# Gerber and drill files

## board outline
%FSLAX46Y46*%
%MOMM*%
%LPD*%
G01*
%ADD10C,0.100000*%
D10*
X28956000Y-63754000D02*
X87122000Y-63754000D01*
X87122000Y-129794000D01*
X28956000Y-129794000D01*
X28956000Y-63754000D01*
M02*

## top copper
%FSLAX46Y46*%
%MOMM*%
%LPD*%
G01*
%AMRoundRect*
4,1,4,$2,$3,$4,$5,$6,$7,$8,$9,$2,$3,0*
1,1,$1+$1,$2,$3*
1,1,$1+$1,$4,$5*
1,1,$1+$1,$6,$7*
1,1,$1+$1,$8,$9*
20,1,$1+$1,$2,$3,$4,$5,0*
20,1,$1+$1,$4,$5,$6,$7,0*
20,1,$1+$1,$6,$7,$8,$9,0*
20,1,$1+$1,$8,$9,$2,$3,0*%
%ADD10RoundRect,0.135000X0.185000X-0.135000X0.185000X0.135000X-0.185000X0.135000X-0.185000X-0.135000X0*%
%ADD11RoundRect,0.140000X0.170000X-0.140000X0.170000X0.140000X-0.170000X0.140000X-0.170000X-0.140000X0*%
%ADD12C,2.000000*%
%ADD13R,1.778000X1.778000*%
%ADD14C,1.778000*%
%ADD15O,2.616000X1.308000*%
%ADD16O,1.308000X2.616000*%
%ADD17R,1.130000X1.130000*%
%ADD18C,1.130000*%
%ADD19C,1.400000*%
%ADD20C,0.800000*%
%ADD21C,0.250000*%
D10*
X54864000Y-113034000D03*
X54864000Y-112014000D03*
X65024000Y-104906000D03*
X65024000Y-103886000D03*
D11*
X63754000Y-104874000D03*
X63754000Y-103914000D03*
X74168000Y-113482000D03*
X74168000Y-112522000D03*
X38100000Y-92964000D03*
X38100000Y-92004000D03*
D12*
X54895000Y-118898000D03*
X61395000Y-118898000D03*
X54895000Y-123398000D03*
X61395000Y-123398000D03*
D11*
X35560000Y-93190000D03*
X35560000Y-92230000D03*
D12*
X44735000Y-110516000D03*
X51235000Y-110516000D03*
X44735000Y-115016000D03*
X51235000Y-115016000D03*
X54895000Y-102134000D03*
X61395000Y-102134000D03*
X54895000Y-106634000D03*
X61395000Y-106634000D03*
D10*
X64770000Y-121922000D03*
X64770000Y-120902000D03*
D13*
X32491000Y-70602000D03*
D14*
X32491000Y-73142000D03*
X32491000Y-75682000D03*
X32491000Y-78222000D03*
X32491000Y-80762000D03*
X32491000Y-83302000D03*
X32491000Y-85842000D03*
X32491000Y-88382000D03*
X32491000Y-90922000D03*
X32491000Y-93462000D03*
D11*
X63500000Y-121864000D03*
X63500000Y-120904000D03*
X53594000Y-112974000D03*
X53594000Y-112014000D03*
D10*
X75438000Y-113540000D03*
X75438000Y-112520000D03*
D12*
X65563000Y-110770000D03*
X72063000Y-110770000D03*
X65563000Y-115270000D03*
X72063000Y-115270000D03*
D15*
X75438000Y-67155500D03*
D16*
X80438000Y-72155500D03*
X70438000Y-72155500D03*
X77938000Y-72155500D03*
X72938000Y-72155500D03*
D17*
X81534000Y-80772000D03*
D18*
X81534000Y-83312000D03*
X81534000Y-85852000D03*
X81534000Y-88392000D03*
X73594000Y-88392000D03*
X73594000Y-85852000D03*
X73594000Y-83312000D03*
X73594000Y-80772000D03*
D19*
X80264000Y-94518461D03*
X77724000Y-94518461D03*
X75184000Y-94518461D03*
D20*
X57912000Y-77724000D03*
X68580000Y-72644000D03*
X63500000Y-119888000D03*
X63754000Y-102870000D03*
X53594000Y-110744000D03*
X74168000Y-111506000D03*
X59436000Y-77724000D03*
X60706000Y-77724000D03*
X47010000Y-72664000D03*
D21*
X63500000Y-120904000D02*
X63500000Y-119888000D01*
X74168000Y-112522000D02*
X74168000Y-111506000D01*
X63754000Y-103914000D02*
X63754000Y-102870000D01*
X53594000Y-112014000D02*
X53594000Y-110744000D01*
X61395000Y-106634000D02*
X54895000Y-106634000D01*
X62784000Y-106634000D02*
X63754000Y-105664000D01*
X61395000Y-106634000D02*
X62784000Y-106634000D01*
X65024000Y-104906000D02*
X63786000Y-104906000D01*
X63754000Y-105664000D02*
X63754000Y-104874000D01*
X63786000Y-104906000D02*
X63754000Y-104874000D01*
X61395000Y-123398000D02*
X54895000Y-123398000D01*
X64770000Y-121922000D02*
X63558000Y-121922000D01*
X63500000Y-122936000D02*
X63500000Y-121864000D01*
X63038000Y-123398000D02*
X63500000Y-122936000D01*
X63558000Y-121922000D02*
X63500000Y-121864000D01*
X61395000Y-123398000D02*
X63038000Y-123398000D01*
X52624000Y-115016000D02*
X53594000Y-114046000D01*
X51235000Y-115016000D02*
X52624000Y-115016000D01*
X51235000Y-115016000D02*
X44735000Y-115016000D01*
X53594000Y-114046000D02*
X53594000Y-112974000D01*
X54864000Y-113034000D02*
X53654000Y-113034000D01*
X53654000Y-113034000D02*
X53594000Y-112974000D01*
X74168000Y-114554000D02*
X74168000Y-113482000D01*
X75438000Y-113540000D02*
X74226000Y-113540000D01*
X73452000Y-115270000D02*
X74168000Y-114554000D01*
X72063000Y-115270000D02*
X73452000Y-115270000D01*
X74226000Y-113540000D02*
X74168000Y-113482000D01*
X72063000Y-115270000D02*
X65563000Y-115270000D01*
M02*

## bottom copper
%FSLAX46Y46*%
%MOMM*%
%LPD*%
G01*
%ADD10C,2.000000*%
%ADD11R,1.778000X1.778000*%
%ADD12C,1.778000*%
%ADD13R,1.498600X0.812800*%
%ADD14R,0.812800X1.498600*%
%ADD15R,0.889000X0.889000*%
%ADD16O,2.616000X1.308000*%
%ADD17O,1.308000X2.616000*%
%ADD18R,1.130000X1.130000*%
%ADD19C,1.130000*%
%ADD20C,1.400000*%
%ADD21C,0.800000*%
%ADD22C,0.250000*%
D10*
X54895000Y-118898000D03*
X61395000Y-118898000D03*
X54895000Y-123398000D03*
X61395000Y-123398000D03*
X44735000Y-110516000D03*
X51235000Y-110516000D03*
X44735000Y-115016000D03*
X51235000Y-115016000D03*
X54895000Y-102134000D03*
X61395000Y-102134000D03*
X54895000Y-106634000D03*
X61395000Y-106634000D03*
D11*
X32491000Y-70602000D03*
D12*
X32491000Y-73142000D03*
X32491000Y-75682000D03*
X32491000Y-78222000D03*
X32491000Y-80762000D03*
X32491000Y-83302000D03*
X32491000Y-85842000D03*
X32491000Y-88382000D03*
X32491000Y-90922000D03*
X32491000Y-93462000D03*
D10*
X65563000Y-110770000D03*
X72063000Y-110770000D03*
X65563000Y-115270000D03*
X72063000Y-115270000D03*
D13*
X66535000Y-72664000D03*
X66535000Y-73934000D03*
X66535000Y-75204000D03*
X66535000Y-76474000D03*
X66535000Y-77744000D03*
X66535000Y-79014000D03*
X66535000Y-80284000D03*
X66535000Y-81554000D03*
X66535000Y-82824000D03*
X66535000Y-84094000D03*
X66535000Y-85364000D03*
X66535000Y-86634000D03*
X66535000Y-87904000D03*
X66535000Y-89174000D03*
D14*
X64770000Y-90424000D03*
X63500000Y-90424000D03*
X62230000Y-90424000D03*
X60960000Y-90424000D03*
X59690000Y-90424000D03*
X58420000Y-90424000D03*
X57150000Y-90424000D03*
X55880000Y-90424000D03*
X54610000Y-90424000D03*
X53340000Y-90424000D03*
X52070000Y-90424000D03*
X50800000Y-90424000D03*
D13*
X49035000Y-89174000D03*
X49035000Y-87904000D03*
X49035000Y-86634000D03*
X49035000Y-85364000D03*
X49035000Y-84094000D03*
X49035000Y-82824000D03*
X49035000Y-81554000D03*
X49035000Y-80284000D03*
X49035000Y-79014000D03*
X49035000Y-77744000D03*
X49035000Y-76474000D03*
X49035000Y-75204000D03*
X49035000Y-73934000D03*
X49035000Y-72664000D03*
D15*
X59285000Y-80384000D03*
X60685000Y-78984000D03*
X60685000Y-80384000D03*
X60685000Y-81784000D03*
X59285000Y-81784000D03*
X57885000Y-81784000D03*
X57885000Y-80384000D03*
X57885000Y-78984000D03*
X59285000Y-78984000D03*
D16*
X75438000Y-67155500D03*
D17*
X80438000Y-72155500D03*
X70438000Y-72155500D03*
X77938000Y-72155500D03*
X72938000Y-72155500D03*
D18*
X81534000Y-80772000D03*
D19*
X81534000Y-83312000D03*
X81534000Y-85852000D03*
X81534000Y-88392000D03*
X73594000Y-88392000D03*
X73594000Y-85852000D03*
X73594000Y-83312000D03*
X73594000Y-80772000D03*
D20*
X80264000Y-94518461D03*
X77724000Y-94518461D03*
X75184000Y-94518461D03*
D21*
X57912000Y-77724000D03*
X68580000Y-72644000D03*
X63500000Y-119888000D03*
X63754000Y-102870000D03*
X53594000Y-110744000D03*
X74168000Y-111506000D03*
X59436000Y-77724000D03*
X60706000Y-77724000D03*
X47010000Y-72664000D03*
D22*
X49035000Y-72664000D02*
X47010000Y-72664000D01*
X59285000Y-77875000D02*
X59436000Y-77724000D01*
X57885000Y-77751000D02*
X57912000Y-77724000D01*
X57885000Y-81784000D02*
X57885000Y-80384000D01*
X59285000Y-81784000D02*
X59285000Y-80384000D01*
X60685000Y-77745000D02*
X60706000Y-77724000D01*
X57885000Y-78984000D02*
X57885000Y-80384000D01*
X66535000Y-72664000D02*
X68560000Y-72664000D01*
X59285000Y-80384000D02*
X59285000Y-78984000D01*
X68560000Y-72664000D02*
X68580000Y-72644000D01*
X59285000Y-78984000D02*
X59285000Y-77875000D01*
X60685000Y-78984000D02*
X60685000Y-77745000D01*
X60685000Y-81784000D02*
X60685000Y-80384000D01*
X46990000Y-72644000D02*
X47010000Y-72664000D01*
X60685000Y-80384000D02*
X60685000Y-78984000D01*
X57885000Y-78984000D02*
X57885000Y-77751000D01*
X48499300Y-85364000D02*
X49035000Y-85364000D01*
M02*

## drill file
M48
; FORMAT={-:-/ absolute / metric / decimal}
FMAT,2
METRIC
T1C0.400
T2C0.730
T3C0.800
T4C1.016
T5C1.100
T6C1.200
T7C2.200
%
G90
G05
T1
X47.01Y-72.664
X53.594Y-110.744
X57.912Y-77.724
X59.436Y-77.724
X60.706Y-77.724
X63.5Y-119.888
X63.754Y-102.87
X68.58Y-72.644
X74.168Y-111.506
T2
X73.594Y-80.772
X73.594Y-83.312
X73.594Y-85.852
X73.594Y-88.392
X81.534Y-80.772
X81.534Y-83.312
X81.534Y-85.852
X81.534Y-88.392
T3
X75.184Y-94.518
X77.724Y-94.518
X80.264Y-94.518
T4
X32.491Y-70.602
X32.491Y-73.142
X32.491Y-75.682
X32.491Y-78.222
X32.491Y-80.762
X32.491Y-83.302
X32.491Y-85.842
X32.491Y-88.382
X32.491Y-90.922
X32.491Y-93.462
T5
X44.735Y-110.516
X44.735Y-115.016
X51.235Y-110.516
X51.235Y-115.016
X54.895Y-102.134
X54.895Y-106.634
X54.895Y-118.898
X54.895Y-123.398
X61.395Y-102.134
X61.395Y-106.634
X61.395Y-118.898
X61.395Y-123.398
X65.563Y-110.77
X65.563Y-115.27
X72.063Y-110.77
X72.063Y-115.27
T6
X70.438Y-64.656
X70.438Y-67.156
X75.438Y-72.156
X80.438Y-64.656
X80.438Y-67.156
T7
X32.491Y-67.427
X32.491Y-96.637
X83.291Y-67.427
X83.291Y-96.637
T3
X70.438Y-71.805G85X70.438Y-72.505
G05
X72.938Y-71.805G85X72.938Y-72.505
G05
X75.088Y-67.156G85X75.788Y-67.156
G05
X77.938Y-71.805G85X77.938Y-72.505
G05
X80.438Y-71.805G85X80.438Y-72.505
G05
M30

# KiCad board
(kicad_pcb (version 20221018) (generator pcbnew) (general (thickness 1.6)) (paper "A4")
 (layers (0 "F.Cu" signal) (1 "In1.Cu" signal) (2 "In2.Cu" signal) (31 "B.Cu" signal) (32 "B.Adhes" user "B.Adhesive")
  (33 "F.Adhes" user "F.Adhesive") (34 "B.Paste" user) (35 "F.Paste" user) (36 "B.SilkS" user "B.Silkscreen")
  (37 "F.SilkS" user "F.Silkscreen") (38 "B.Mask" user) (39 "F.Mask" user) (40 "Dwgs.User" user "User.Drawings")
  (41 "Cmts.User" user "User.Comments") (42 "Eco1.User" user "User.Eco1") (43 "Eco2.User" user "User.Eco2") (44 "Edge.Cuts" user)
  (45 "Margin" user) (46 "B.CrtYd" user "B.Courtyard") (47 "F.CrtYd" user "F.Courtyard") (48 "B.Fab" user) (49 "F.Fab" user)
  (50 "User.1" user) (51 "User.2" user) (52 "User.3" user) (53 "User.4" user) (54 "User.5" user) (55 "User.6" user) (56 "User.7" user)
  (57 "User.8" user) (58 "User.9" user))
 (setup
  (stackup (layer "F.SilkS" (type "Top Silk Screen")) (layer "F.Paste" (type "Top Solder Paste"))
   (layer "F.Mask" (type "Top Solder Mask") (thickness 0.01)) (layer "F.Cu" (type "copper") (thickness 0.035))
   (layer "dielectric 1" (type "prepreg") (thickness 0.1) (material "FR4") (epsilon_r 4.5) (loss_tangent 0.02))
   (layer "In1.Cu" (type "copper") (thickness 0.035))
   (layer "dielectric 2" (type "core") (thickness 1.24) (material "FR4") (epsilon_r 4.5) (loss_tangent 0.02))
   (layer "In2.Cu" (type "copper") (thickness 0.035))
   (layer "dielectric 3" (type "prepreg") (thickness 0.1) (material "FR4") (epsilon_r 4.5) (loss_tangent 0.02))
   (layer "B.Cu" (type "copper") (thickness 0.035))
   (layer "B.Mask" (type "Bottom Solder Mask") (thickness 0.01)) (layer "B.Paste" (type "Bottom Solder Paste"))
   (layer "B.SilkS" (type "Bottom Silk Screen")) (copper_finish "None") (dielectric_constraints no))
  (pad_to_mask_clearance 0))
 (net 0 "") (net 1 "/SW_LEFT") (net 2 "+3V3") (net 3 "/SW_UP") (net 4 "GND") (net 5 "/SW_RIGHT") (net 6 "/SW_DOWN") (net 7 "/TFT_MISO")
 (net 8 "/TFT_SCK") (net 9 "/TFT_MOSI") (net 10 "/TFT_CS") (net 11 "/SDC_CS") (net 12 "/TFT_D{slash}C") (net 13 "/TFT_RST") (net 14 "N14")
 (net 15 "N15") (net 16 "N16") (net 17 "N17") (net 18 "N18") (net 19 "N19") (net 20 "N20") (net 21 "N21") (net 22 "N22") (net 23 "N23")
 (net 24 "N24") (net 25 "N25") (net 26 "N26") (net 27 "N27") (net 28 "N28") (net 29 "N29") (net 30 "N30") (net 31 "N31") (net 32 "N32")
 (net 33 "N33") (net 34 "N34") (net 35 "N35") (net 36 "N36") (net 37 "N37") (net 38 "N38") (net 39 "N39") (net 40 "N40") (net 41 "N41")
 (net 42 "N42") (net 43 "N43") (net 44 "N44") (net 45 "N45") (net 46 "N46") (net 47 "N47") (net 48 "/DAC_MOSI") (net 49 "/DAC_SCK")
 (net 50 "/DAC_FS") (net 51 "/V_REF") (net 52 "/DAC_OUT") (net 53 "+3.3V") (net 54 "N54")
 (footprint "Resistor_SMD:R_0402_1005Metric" (layer "F.Cu") (at 54.864 112.524 90)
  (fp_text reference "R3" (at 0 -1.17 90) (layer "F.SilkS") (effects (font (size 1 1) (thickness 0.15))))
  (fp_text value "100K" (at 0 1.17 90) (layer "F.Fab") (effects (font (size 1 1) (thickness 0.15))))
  (pad "1" smd roundrect (at -0.51 0 90) (size 0.54 0.64) (layers "F.Cu" "F.Paste" "F.Mask") (roundrect_rratio 0.25) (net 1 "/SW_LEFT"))
  (pad "2" smd roundrect (at 0.51 0 90) (size 0.54 0.64) (layers "F.Cu" "F.Paste" "F.Mask") (roundrect_rratio 0.25) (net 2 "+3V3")))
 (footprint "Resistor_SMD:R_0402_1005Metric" (layer "F.Cu") (at 65.024 104.396 90)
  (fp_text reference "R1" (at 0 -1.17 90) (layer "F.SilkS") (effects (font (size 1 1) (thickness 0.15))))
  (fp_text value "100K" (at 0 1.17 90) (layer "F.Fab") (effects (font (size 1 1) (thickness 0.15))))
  (pad "1" smd roundrect (at -0.51 0 90) (size 0.54 0.64) (layers "F.Cu" "F.Paste" "F.Mask") (roundrect_rratio 0.25) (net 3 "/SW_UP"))
  (pad "2" smd roundrect (at 0.51 0 90) (size 0.54 0.64) (layers "F.Cu" "F.Paste" "F.Mask") (roundrect_rratio 0.25) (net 2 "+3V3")))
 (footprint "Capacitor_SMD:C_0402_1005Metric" (layer "F.Cu") (at 63.754 104.394 90)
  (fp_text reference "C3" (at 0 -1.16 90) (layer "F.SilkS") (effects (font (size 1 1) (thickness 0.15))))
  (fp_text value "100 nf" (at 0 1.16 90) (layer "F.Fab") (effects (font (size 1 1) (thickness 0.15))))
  (pad "1" smd roundrect (at -0.48 0 90) (size 0.56 0.62) (layers "F.Cu" "F.Paste" "F.Mask") (roundrect_rratio 0.25) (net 3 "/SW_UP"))
  (pad "2" smd roundrect (at 0.48 0 90) (size 0.56 0.62) (layers "F.Cu" "F.Paste" "F.Mask") (roundrect_rratio 0.25) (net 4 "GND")))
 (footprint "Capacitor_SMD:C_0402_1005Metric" (layer "F.Cu") (at 74.168 113.002 90)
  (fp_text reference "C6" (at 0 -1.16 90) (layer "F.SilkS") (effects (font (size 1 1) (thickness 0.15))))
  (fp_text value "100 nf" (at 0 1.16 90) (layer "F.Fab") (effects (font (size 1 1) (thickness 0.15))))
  (pad "1" smd roundrect (at -0.48 0 90) (size 0.56 0.62) (layers "F.Cu" "F.Paste" "F.Mask") (roundrect_rratio 0.25) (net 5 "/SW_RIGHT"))
  (pad "2" smd roundrect (at 0.48 0 90) (size 0.56 0.62) (layers "F.Cu" "F.Paste" "F.Mask") (roundrect_rratio 0.25) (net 4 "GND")))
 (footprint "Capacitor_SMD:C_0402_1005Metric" (layer "F.Cu") (at 38.1 92.484 90)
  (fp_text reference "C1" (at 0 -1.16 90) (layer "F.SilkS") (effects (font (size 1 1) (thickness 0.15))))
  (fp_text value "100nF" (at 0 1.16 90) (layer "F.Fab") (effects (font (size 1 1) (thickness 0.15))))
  (pad "1" smd roundrect (at -0.48 0 90) (size 0.56 0.62) (layers "F.Cu" "F.Paste" "F.Mask") (roundrect_rratio 0.25) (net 2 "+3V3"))
  (pad "2" smd roundrect (at 0.48 0 90) (size 0.56 0.62) (layers "F.Cu" "F.Paste" "F.Mask") (roundrect_rratio 0.25) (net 4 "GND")))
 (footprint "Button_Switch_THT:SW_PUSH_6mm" (layer "F.Cu") (at 54.895 118.898)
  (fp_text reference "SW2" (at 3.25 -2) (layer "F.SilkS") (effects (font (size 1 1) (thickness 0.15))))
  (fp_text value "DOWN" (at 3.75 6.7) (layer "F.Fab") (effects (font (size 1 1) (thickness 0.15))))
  (pad "1" thru_hole circle (at 0 0 90) (size 2 2) (drill 1.1) (layers "*.Cu" "*.Mask") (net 4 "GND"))
  (pad "1" thru_hole circle (at 6.5 0 90) (size 2 2) (drill 1.1) (layers "*.Cu" "*.Mask") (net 4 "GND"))
  (pad "2" thru_hole circle (at 0 4.5 90) (size 2 2) (drill 1.1) (layers "*.Cu" "*.Mask") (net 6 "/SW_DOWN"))
  (pad "2" thru_hole circle (at 6.5 4.5 90) (size 2 2) (drill 1.1) (layers "*.Cu" "*.Mask") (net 6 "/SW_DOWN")))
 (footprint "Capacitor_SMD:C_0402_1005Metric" (layer "F.Cu") (at 35.56 92.71 90)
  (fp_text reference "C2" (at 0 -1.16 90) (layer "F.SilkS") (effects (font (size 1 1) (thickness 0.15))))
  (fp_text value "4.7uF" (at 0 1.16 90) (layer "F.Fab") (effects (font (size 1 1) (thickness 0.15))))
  (pad "1" smd roundrect (at -0.48 0 90) (size 0.56 0.62) (layers "F.Cu" "F.Paste" "F.Mask") (roundrect_rratio 0.25) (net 2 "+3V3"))
  (pad "2" smd roundrect (at 0.48 0 90) (size 0.56 0.62) (layers "F.Cu" "F.Paste" "F.Mask") (roundrect_rratio 0.25) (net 4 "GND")))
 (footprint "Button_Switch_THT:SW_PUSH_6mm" (layer "F.Cu") (at 44.735 110.516)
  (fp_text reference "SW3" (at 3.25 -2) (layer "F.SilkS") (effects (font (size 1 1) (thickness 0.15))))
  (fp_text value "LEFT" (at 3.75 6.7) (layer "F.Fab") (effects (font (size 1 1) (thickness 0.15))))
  (pad "1" thru_hole circle (at 0 0 90) (size 2 2) (drill 1.1) (layers "*.Cu" "*.Mask") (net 4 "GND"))
  (pad "1" thru_hole circle (at 6.5 0 90) (size 2 2) (drill 1.1) (layers "*.Cu" "*.Mask") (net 4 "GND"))
  (pad "2" thru_hole circle (at 0 4.5 90) (size 2 2) (drill 1.1) (layers "*.Cu" "*.Mask") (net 1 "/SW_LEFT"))
  (pad "2" thru_hole circle (at 6.5 4.5 90) (size 2 2) (drill 1.1) (layers "*.Cu" "*.Mask") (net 1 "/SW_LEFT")))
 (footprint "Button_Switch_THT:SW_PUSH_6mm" (layer "F.Cu") (at 54.895 102.134)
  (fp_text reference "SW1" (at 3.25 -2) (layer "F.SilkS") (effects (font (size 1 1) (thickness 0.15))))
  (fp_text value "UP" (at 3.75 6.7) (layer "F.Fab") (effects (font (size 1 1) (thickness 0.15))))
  (pad "1" thru_hole circle (at 0 0 90) (size 2 2) (drill 1.1) (layers "*.Cu" "*.Mask") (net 4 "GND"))
  (pad "1" thru_hole circle (at 6.5 0 90) (size 2 2) (drill 1.1) (layers "*.Cu" "*.Mask") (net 4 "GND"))
  (pad "2" thru_hole circle (at 0 4.5 90) (size 2 2) (drill 1.1) (layers "*.Cu" "*.Mask") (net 3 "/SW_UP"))
  (pad "2" thru_hole circle (at 6.5 4.5 90) (size 2 2) (drill 1.1) (layers "*.Cu" "*.Mask") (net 3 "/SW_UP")))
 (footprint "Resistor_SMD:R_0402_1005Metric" (layer "F.Cu") (at 64.77 121.412 90)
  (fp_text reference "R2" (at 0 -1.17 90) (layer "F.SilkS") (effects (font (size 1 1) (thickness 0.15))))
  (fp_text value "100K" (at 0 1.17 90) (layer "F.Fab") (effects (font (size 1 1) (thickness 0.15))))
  (pad "1" smd roundrect (at -0.51 0 90) (size 0.54 0.64) (layers "F.Cu" "F.Paste" "F.Mask") (roundrect_rratio 0.25) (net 6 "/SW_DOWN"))
  (pad "2" smd roundrect (at 0.51 0 90) (size 0.54 0.64) (layers "F.Cu" "F.Paste" "F.Mask") (roundrect_rratio 0.25) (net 2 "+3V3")))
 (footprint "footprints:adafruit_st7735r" (layer "F.Cu") (at 57.891 82.032)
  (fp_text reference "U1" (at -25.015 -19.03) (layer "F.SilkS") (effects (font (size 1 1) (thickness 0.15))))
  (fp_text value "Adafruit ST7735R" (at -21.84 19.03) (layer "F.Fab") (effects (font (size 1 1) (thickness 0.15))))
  (pad "" np_thru_hole circle (at -25.4 -14.605) (size 2.2 2.2) (drill 2.2) (layers "*.Cu" "*.Mask"))
  (pad "" np_thru_hole circle (at -25.4 14.605) (size 2.2 2.2) (drill 2.2) (layers "*.Cu" "*.Mask"))
  (pad "" np_thru_hole circle (at 25.4 -14.605) (size 2.2 2.2) (drill 2.2) (layers "*.Cu" "*.Mask"))
  (pad "" np_thru_hole circle (at 25.4 14.605) (size 2.2 2.2) (drill 2.2) (layers "*.Cu" "*.Mask"))
  (pad "1" thru_hole rect (at -25.4 -11.43) (size 1.778 1.778) (drill 1.016) (layers "*.Cu" "*.Mask") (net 2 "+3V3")
   (solder_mask_margin 0.102))
  (pad "2" thru_hole circle (at -25.4 -8.89) (size 1.778 1.778) (drill 1.016) (layers "*.Cu" "*.Mask") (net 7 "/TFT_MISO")
   (solder_mask_margin 0.102))
  (pad "3" thru_hole circle (at -25.4 -6.35) (size 1.778 1.778) (drill 1.016) (layers "*.Cu" "*.Mask") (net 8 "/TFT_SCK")
   (solder_mask_margin 0.102))
  (pad "4" thru_hole circle (at -25.4 -3.81) (size 1.778 1.778) (drill 1.016) (layers "*.Cu" "*.Mask") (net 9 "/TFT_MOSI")
   (solder_mask_margin 0.102))
  (pad "5" thru_hole circle (at -25.4 -1.27) (size 1.778 1.778) (drill 1.016) (layers "*.Cu" "*.Mask") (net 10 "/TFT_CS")
   (solder_mask_margin 0.102))
  (pad "6" thru_hole circle (at -25.4 1.27) (size 1.778 1.778) (drill 1.016) (layers "*.Cu" "*.Mask") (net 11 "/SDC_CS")
   (solder_mask_margin 0.102))
  (pad "7" thru_hole circle (at -25.4 3.81) (size 1.778 1.778) (drill 1.016) (layers "*.Cu" "*.Mask") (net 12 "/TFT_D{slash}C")
   (solder_mask_margin 0.102))
  (pad "8" thru_hole circle (at -25.4 6.35) (size 1.778 1.778) (drill 1.016) (layers "*.Cu" "*.Mask") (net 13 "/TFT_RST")
   (solder_mask_margin 0.102))
  (pad "9" thru_hole circle (at -25.4 8.89) (size 1.778 1.778) (drill 1.016) (layers "*.Cu" "*.Mask") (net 2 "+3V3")
   (solder_mask_margin 0.102))
  (pad "10" thru_hole circle (at -25.4 11.43) (size 1.778 1.778) (drill 1.016) (layers "*.Cu" "*.Mask") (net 4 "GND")
   (solder_mask_margin 0.102)))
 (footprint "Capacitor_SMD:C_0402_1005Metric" (layer "F.Cu") (at 63.5 121.384 90)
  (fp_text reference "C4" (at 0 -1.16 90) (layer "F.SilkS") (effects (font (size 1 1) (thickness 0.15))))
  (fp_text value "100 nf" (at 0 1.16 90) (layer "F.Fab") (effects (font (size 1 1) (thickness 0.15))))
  (pad "1" smd roundrect (at -0.48 0 90) (size 0.56 0.62) (layers "F.Cu" "F.Paste" "F.Mask") (roundrect_rratio 0.25) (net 6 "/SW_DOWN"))
  (pad "2" smd roundrect (at 0.48 0 90) (size 0.56 0.62) (layers "F.Cu" "F.Paste" "F.Mask") (roundrect_rratio 0.25) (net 4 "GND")))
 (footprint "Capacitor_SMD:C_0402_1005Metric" (layer "F.Cu") (at 53.594 112.494 90)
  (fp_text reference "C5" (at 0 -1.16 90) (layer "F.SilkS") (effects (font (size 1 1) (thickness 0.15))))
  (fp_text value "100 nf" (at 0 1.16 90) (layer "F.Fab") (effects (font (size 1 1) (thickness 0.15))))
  (pad "1" smd roundrect (at -0.48 0 90) (size 0.56 0.62) (layers "F.Cu" "F.Paste" "F.Mask") (roundrect_rratio 0.25) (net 1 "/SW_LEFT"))
  (pad "2" smd roundrect (at 0.48 0 90) (size 0.56 0.62) (layers "F.Cu" "F.Paste" "F.Mask") (roundrect_rratio 0.25) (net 4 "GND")))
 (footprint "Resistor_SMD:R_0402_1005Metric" (layer "F.Cu") (at 75.438 113.03 90)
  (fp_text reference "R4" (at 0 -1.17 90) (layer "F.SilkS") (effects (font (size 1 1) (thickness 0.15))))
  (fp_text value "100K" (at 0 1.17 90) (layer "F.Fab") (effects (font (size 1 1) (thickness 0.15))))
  (pad "1" smd roundrect (at -0.51 0 90) (size 0.54 0.64) (layers "F.Cu" "F.Paste" "F.Mask") (roundrect_rratio 0.25) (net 5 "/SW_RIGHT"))
  (pad "2" smd roundrect (at 0.51 0 90) (size 0.54 0.64) (layers "F.Cu" "F.Paste" "F.Mask") (roundrect_rratio 0.25) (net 2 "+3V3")))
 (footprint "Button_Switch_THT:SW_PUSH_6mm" (layer "F.Cu") (at 65.563 110.77)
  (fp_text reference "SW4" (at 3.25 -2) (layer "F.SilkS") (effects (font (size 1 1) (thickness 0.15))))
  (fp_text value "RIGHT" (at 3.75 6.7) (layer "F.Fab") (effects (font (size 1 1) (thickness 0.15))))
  (pad "1" thru_hole circle (at 0 0 90) (size 2 2) (drill 1.1) (layers "*.Cu" "*.Mask") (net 4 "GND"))
  (pad "1" thru_hole circle (at 6.5 0 90) (size 2 2) (drill 1.1) (layers "*.Cu" "*.Mask") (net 4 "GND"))
  (pad "2" thru_hole circle (at 0 4.5 90) (size 2 2) (drill 1.1) (layers "*.Cu" "*.Mask") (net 5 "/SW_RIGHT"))
  (pad "2" thru_hole circle (at 6.5 4.5 90) (size 2 2) (drill 1.1) (layers "*.Cu" "*.Mask") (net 5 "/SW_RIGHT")))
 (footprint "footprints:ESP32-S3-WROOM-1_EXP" (layer "B.Cu") (at 57.785 77.924 180)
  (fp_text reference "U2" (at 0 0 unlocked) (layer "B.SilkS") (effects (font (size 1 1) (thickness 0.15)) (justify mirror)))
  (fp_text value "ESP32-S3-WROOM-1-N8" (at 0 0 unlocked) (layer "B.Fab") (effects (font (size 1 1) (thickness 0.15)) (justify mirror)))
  (pad "1" smd rect (at -8.75 5.26 180) (size 1.4986 0.8128) (layers "B.Cu" "B.Paste" "B.Mask") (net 4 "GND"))
  (pad "2" smd rect (at -8.75 3.99 180) (size 1.4986 0.8128) (layers "B.Cu" "B.Paste" "B.Mask") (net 2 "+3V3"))
  (pad "3" smd rect (at -8.75 2.72 180) (size 1.4986 0.8128) (layers "B.Cu" "B.Paste" "B.Mask") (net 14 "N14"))
  (pad "4" smd rect (at -8.75 1.45 180) (size 1.4986 0.8128) (layers "B.Cu" "B.Paste" "B.Mask") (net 13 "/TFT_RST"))
  (pad "5" smd rect (at -8.75 0.18 180) (size 1.4986 0.8128) (layers "B.Cu" "B.Paste" "B.Mask") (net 10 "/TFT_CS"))
  (pad "6" smd rect (at -8.75 -1.09 180) (size 1.4986 0.8128) (layers "B.Cu" "B.Paste" "B.Mask") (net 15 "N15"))
  (pad "7" smd rect (at -8.75 -2.36 180) (size 1.4986 0.8128) (layers "B.Cu" "B.Paste" "B.Mask") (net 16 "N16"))
  (pad "8" smd rect (at -8.75 -3.63 180) (size 1.4986 0.8128) (layers "B.Cu" "B.Paste" "B.Mask") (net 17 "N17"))
  (pad "9" smd rect (at -8.75 -4.9 180) (size 1.4986 0.8128) (layers "B.Cu" "B.Paste" "B.Mask") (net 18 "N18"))
  (pad "10" smd rect (at -8.75 -6.17 180) (size 1.4986 0.8128) (layers "B.Cu" "B.Paste" "B.Mask") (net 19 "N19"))
  (pad "11" smd rect (at -8.75 -7.44 180) (size 1.4986 0.8128) (layers "B.Cu" "B.Paste" "B.Mask") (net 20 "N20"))
  (pad "12" smd rect (at -8.75 -8.71 180) (size 1.4986 0.8128) (layers "B.Cu" "B.Paste" "B.Mask") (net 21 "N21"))
  (pad "13" smd rect (at -8.75 -9.98 180) (size 1.4986 0.8128) (layers "B.Cu" "B.Paste" "B.Mask") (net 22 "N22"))
  (pad "14" smd rect (at -8.75 -11.25 180) (size 1.4986 0.8128) (layers "B.Cu" "B.Paste" "B.Mask") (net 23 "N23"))
  (pad "15" smd rect (at -6.985 -12.5 90) (size 1.4986 0.8128) (layers "B.Cu" "B.Paste" "B.Mask") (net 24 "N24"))
  (pad "16" smd rect (at -5.715 -12.5 90) (size 1.4986 0.8128) (layers "B.Cu" "B.Paste" "B.Mask") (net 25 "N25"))
  (pad "17" smd rect (at -4.445 -12.5 90) (size 1.4986 0.8128) (layers "B.Cu" "B.Paste" "B.Mask") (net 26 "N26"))
  (pad "18" smd rect (at -3.175 -12.5 90) (size 1.4986 0.8128) (layers "B.Cu" "B.Paste" "B.Mask") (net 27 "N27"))
  (pad "19" smd rect (at -1.905 -12.5 90) (size 1.4986 0.8128) (layers "B.Cu" "B.Paste" "B.Mask") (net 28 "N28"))
  (pad "20" smd rect (at -0.635 -12.5 90) (size 1.4986 0.8128) (layers "B.Cu" "B.Paste" "B.Mask") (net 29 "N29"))
  (pad "21" smd rect (at 0.635 -12.5 90) (size 1.4986 0.8128) (layers "B.Cu" "B.Paste" "B.Mask") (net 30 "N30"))
  (pad "22" smd rect (at 1.905 -12.5 90) (size 1.4986 0.8128) (layers "B.Cu" "B.Paste" "B.Mask") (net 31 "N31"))
  (pad "23" smd rect (at 3.175 -12.5 90) (size 1.4986 0.8128) (layers "B.Cu" "B.Paste" "B.Mask") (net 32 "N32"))
  (pad "24" smd rect (at 4.445 -12.5 90) (size 1.4986 0.8128) (layers "B.Cu" "B.Paste" "B.Mask") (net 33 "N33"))
  (pad "25" smd rect (at 5.715 -12.5 90) (size 1.4986 0.8128) (layers "B.Cu" "B.Paste" "B.Mask") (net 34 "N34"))
  (pad "26" smd rect (at 6.985 -12.5 90) (size 1.4986 0.8128) (layers "B.Cu" "B.Paste" "B.Mask") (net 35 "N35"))
  (pad "27" smd rect (at 8.75 -11.25 180) (size 1.4986 0.8128) (layers "B.Cu" "B.Paste" "B.Mask") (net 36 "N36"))
  (pad "28" smd rect (at 8.75 -9.98 180) (size 1.4986 0.8128) (layers "B.Cu" "B.Paste" "B.Mask") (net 9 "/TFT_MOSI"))
  (pad "29" smd rect (at 8.75 -8.71 180) (size 1.4986 0.8128) (layers "B.Cu" "B.Paste" "B.Mask") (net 8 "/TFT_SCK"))
  (pad "30" smd rect (at 8.75 -7.44 180) (size 1.4986 0.8128) (layers "B.Cu" "B.Paste" "B.Mask") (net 7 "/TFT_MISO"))
  (pad "31" smd rect (at 8.75 -6.17 180) (size 1.4986 0.8128) (layers "B.Cu" "B.Paste" "B.Mask") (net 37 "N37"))
  (pad "32" smd rect (at 8.75 -4.9 180) (size 1.4986 0.8128) (layers "B.Cu" "B.Paste" "B.Mask") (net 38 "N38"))
  (pad "33" smd rect (at 8.75 -3.63 180) (size 1.4986 0.8128) (layers "B.Cu" "B.Paste" "B.Mask") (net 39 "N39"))
  (pad "34" smd rect (at 8.75 -2.36 180) (size 1.4986 0.8128) (layers "B.Cu" "B.Paste" "B.Mask") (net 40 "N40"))
  (pad "35" smd rect (at 8.75 -1.09 180) (size 1.4986 0.8128) (layers "B.Cu" "B.Paste" "B.Mask") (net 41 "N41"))
  (pad "36" smd rect (at 8.75 0.18 180) (size 1.4986 0.8128) (layers "B.Cu" "B.Paste" "B.Mask") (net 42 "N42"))
  (pad "37" smd rect (at 8.75 1.45 180) (size 1.4986 0.8128) (layers "B.Cu" "B.Paste" "B.Mask") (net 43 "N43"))
  (pad "38" smd rect (at 8.75 2.72 180) (size 1.4986 0.8128) (layers "B.Cu" "B.Paste" "B.Mask") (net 12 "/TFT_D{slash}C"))
  (pad "39" smd rect (at 8.75 3.99 180) (size 1.4986 0.8128) (layers "B.Cu" "B.Paste" "B.Mask") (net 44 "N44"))
  (pad "40" smd rect (at 8.75 5.26 180) (size 1.4986 0.8128) (layers "B.Cu" "B.Paste" "B.Mask") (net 4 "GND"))
  (pad "41" smd rect (at -1.5 -2.46 180) (size 0.889 0.889) (layers "B.Cu" "B.Paste" "B.Mask") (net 4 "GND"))
  (pad "42" smd rect (at -2.9 -1.06 180) (size 0.889 0.889) (layers "B.Cu" "B.Paste" "B.Mask") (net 4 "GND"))
  (pad "43" smd rect (at -2.9 -2.46 180) (size 0.889 0.889) (layers "B.Cu" "B.Paste" "B.Mask") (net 4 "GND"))
  (pad "44" smd rect (at -2.9 -3.86 180) (size 0.889 0.889) (layers "B.Cu" "B.Paste" "B.Mask") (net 4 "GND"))
  (pad "45" smd rect (at -1.5 -3.86 180) (size 0.889 0.889) (layers "B.Cu" "B.Paste" "B.Mask") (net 4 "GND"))
  (pad "46" smd rect (at -0.1 -3.86 180) (size 0.889 0.889) (layers "B.Cu" "B.Paste" "B.Mask") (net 4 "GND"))
  (pad "47" smd rect (at -0.1 -2.46 180) (size 0.889 0.889) (layers "B.Cu" "B.Paste" "B.Mask") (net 4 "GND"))
  (pad "48" smd rect (at -0.1 -1.06 180) (size 0.889 0.889) (layers "B.Cu" "B.Paste" "B.Mask") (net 4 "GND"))
  (pad "49" smd rect (at -1.5 -1.06 180) (size 0.889 0.889) (layers "B.Cu" "B.Paste" "B.Mask") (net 4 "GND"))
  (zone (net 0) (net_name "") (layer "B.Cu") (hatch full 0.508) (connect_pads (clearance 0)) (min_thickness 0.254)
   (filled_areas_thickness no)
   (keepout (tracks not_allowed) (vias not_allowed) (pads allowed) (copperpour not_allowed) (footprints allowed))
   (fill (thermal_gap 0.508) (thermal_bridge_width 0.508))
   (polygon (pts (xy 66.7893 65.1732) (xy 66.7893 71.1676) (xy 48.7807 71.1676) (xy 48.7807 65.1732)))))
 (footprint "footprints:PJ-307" (layer "B.Cu") (at 75.438 67.1555)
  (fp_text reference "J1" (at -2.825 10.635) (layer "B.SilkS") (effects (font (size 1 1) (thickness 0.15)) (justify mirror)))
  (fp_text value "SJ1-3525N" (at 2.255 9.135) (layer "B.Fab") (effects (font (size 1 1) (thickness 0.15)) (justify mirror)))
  (pad "" np_thru_hole circle (at -5 -2.5) (size 1.2 1.2) (drill 1.2) (layers "*.Cu" "*.Mask"))
  (pad "" np_thru_hole circle (at -5 0) (size 1.2 1.2) (drill 1.2) (layers "*.Cu" "*.Mask"))
  (pad "" np_thru_hole circle (at 0 5) (size 1.2 1.2) (drill 1.2) (layers "*.Cu" "*.Mask"))
  (pad "" np_thru_hole circle (at 5 -2.5) (size 1.2 1.2) (drill 1.2) (layers "*.Cu" "*.Mask"))
  (pad "" np_thru_hole circle (at 5 0) (size 1.2 1.2) (drill 1.2) (layers "*.Cu" "*.Mask"))
  (pad "1" thru_hole oval (at 0 0) (size 2.616 1.308) (drill oval 1.5 0.8) (layers "*.Cu" "*.Mask") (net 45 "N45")
   (solder_mask_margin 0.102))
  (pad "2" thru_hole oval (at 5 5) (size 1.308 2.616) (drill oval 0.8 1.5) (layers "*.Cu" "*.Mask") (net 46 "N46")
   (solder_mask_margin 0.102))
  (pad "3" thru_hole oval (at -5 5) (size 1.308 2.616) (drill oval 0.8 1.5) (layers "*.Cu" "*.Mask") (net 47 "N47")
   (solder_mask_margin 0.102))
  (pad "10" thru_hole oval (at 2.5 5) (size 1.308 2.616) (drill oval 0.8 1.5) (layers "*.Cu" "*.Mask") (solder_mask_margin 0.102))
  (pad "11" thru_hole oval (at -2.5 5) (size 1.308 2.616) (drill oval 0.8 1.5) (layers "*.Cu" "*.Mask") (solder_mask_margin 0.102)))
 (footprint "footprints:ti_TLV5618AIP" (layer "B.Cu") (at 77.564 84.582 180)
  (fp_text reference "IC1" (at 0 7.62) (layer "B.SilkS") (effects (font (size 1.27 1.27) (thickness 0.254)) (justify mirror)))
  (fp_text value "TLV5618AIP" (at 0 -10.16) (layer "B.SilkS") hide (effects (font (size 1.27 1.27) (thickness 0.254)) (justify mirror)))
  (pad "1" thru_hole rect (at -3.97 3.81 180) (size 1.13 1.13) (drill 0.73) (layers "*.Cu" "*.Mask") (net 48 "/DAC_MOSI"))
  (pad "2" thru_hole circle (at -3.97 1.27 180) (size 1.13 1.13) (drill 0.73) (layers "*.Cu" "*.Mask") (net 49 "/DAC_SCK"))
  (pad "3" thru_hole circle (at -3.97 -1.27 180) (size 1.13 1.13) (drill 0.73) (layers "*.Cu" "*.Mask") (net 4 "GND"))
  (pad "4" thru_hole circle (at -3.97 -3.81 180) (size 1.13 1.13) (drill 0.73) (layers "*.Cu" "*.Mask") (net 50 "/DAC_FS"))
  (pad "5" thru_hole circle (at 3.97 -3.81 180) (size 1.13 1.13) (drill 0.73) (layers "*.Cu" "*.Mask") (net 4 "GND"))
  (pad "6" thru_hole circle (at 3.97 -1.27 180) (size 1.13 1.13) (drill 0.73) (layers "*.Cu" "*.Mask") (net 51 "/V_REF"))
  (pad "7" thru_hole circle (at 3.97 1.27 180) (size 1.13 1.13) (drill 0.73) (layers "*.Cu" "*.Mask") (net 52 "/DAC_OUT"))
  (pad "8" thru_hole circle (at 3.97 3.81 180) (size 1.13 1.13) (drill 0.73) (layers "*.Cu" "*.Mask") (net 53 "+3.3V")))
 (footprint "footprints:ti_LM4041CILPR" (layer "B.Cu") (at 77.724 94.518461 180)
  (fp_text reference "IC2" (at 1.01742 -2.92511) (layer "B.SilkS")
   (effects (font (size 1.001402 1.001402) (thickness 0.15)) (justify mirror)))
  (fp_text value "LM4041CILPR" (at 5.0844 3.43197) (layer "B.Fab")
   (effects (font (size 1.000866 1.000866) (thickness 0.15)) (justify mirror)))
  (pad "1" thru_hole circle (at -2.54 0 180) (size 1.4 1.4) (drill 0.8) (layers "*.Cu" "*.Mask") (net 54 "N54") (solder_mask_margin 0.102))
  (pad "2" thru_hole circle (at 0 0 180) (size 1.4 1.4) (drill 0.8) (layers "*.Cu" "*.Mask") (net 51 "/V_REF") (solder_mask_margin 0.102))
  (pad "3" thru_hole circle (at 2.54 0 180) (size 1.4 1.4) (drill 0.8) (layers "*.Cu" "*.Mask") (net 4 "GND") (solder_mask_margin 0.102)))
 (gr_rect (start 28.956 63.754) (end 87.122 129.794) (stroke (width 0.1) (type default)) (fill none) (layer "Edge.Cuts"))
 (segment (start 63.5 120.904) (end 63.5 119.888) (width 0.25) (layer "F.Cu") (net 4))
 (segment (start 74.168 112.522) (end 74.168 111.506) (width 0.25) (layer "F.Cu") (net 4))
 (segment (start 63.754 103.914) (end 63.754 102.87) (width 0.25) (layer "F.Cu") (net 4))
 (segment (start 53.594 112.014) (end 53.594 110.744) (width 0.25) (layer "F.Cu") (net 4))
 (via (at 57.912 77.724) (size 0.8) (drill 0.4) (layers "F.Cu" "B.Cu") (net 4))
 (via (at 68.58 72.644) (size 0.8) (drill 0.4) (layers "F.Cu" "B.Cu") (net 4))
 (via (at 63.5 119.888) (size 0.8) (drill 0.4) (layers "F.Cu" "B.Cu") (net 4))
 (via (at 63.754 102.87) (size 0.8) (drill 0.4) (layers "F.Cu" "B.Cu") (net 4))
 (via (at 53.594 110.744) (size 0.8) (drill 0.4) (layers "F.Cu" "B.Cu") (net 4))
 (via (at 74.168 111.506) (size 0.8) (drill 0.4) (layers "F.Cu" "B.Cu") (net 4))
 (via (at 59.436 77.724) (size 0.8) (drill 0.4) (layers "F.Cu" "B.Cu") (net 4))
 (via (at 60.706 77.724) (size 0.8) (drill 0.4) (layers "F.Cu" "B.Cu") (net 4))
 (via (at 47.01 72.664) (size 0.8) (drill 0.4) (layers "F.Cu" "B.Cu") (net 4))
 (segment (start 49.035 72.664) (end 47.01 72.664) (width 0.25) (layer "B.Cu") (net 4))
 (segment (start 59.285 77.875) (end 59.436 77.724) (width 0.25) (layer "B.Cu") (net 4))
 (segment (start 57.885 77.751) (end 57.912 77.724) (width 0.25) (layer "B.Cu") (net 4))
 (segment (start 57.885 81.784) (end 57.885 80.384) (width 0.25) (layer "B.Cu") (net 4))
 (segment (start 59.285 81.784) (end 59.285 80.384) (width 0.25) (layer "B.Cu") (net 4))
 (segment (start 60.685 77.745) (end 60.706 77.724) (width 0.25) (layer "B.Cu") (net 4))
 (segment (start 57.885 78.984) (end 57.885 80.384) (width 0.25) (layer "B.Cu") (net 4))
 (segment (start 66.535 72.664) (end 68.56 72.664) (width 0.25) (layer "B.Cu") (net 4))
 (segment (start 59.285 80.384) (end 59.285 78.984) (width 0.25) (layer "B.Cu") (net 4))
 (segment (start 68.56 72.664) (end 68.58 72.644) (width 0.25) (layer "B.Cu") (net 4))
 (segment (start 59.285 78.984) (end 59.285 77.875) (width 0.25) (layer "B.Cu") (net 4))
 (segment (start 60.685 78.984) (end 60.685 77.745) (width 0.25) (layer "B.Cu") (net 4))
 (segment (start 60.685 81.784) (end 60.685 80.384) (width 0.25) (layer "B.Cu") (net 4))
 (segment (start 46.99 72.644) (end 47.01 72.664) (width 0.25) (layer "B.Cu") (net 4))
 (segment (start 60.685 80.384) (end 60.685 78.984) (width 0.25) (layer "B.Cu") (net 4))
 (segment (start 57.885 78.984) (end 57.885 77.751) (width 0.25) (layer "B.Cu") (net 4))
 (segment (start 48.4993 85.364) (end 49.035 85.364) (width 0.25) (layer "B.Cu") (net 7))
 (segment (start 61.395 106.634) (end 54.895 106.634) (width 0.25) (layer "F.Cu") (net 3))
 (segment (start 62.784 106.634) (end 63.754 105.664) (width 0.25) (layer "F.Cu") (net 3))
 (segment (start 61.395 106.634) (end 62.784 106.634) (width 0.25) (layer "F.Cu") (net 3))
 (segment (start 65.024 104.906) (end 63.786 104.906) (width 0.25) (layer "F.Cu") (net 3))
 (segment (start 63.754 105.664) (end 63.754 104.874) (width 0.25) (layer "F.Cu") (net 3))
 (segment (start 63.786 104.906) (end 63.754 104.874) (width 0.25) (layer "F.Cu") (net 3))
 (segment (start 61.395 123.398) (end 54.895 123.398) (width 0.25) (layer "F.Cu") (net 6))
 (segment (start 64.77 121.922) (end 63.558 121.922) (width 0.25) (layer "F.Cu") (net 6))
 (segment (start 63.5 122.936) (end 63.5 121.864) (width 0.25) (layer "F.Cu") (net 6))
 (segment (start 63.038 123.398) (end 63.5 122.936) (width 0.25) (layer "F.Cu") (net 6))
 (segment (start 63.558 121.922) (end 63.5 121.864) (width 0.25) (layer "F.Cu") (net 6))
 (segment (start 61.395 123.398) (end 63.038 123.398) (width 0.25) (layer "F.Cu") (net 6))
 (segment (start 52.624 115.016) (end 53.594 114.046) (width 0.25) (layer "F.Cu") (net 1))
 (segment (start 51.235 115.016) (end 52.624 115.016) (width 0.25) (layer "F.Cu") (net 1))
 (segment (start 51.235 115.016) (end 44.735 115.016) (width 0.25) (layer "F.Cu") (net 1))
 (segment (start 53.594 114.046) (end 53.594 112.974) (width 0.25) (layer "F.Cu") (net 1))
 (segment (start 54.864 113.034) (end 53.654 113.034) (width 0.25) (layer "F.Cu") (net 1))
 (segment (start 53.654 113.034) (end 53.594 112.974) (width 0.25) (layer "F.Cu") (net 1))
 (segment (start 74.168 114.554) (end 74.168 113.482) (width 0.25) (layer "F.Cu") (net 5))
 (segment (start 75.438 113.54) (end 74.226 113.54) (width 0.25) (layer "F.Cu") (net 5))
 (segment (start 73.452 115.27) (end 74.168 114.554) (width 0.25) (layer "F.Cu") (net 5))
 (segment (start 72.063 115.27) (end 73.452 115.27) (width 0.25) (layer "F.Cu") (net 5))
 (segment (start 74.226 113.54) (end 74.168 113.482) (width 0.25) (layer "F.Cu") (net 5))
 (segment (start 72.063 115.27) (end 65.563 115.27) (width 0.25) (layer "F.Cu") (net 5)))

